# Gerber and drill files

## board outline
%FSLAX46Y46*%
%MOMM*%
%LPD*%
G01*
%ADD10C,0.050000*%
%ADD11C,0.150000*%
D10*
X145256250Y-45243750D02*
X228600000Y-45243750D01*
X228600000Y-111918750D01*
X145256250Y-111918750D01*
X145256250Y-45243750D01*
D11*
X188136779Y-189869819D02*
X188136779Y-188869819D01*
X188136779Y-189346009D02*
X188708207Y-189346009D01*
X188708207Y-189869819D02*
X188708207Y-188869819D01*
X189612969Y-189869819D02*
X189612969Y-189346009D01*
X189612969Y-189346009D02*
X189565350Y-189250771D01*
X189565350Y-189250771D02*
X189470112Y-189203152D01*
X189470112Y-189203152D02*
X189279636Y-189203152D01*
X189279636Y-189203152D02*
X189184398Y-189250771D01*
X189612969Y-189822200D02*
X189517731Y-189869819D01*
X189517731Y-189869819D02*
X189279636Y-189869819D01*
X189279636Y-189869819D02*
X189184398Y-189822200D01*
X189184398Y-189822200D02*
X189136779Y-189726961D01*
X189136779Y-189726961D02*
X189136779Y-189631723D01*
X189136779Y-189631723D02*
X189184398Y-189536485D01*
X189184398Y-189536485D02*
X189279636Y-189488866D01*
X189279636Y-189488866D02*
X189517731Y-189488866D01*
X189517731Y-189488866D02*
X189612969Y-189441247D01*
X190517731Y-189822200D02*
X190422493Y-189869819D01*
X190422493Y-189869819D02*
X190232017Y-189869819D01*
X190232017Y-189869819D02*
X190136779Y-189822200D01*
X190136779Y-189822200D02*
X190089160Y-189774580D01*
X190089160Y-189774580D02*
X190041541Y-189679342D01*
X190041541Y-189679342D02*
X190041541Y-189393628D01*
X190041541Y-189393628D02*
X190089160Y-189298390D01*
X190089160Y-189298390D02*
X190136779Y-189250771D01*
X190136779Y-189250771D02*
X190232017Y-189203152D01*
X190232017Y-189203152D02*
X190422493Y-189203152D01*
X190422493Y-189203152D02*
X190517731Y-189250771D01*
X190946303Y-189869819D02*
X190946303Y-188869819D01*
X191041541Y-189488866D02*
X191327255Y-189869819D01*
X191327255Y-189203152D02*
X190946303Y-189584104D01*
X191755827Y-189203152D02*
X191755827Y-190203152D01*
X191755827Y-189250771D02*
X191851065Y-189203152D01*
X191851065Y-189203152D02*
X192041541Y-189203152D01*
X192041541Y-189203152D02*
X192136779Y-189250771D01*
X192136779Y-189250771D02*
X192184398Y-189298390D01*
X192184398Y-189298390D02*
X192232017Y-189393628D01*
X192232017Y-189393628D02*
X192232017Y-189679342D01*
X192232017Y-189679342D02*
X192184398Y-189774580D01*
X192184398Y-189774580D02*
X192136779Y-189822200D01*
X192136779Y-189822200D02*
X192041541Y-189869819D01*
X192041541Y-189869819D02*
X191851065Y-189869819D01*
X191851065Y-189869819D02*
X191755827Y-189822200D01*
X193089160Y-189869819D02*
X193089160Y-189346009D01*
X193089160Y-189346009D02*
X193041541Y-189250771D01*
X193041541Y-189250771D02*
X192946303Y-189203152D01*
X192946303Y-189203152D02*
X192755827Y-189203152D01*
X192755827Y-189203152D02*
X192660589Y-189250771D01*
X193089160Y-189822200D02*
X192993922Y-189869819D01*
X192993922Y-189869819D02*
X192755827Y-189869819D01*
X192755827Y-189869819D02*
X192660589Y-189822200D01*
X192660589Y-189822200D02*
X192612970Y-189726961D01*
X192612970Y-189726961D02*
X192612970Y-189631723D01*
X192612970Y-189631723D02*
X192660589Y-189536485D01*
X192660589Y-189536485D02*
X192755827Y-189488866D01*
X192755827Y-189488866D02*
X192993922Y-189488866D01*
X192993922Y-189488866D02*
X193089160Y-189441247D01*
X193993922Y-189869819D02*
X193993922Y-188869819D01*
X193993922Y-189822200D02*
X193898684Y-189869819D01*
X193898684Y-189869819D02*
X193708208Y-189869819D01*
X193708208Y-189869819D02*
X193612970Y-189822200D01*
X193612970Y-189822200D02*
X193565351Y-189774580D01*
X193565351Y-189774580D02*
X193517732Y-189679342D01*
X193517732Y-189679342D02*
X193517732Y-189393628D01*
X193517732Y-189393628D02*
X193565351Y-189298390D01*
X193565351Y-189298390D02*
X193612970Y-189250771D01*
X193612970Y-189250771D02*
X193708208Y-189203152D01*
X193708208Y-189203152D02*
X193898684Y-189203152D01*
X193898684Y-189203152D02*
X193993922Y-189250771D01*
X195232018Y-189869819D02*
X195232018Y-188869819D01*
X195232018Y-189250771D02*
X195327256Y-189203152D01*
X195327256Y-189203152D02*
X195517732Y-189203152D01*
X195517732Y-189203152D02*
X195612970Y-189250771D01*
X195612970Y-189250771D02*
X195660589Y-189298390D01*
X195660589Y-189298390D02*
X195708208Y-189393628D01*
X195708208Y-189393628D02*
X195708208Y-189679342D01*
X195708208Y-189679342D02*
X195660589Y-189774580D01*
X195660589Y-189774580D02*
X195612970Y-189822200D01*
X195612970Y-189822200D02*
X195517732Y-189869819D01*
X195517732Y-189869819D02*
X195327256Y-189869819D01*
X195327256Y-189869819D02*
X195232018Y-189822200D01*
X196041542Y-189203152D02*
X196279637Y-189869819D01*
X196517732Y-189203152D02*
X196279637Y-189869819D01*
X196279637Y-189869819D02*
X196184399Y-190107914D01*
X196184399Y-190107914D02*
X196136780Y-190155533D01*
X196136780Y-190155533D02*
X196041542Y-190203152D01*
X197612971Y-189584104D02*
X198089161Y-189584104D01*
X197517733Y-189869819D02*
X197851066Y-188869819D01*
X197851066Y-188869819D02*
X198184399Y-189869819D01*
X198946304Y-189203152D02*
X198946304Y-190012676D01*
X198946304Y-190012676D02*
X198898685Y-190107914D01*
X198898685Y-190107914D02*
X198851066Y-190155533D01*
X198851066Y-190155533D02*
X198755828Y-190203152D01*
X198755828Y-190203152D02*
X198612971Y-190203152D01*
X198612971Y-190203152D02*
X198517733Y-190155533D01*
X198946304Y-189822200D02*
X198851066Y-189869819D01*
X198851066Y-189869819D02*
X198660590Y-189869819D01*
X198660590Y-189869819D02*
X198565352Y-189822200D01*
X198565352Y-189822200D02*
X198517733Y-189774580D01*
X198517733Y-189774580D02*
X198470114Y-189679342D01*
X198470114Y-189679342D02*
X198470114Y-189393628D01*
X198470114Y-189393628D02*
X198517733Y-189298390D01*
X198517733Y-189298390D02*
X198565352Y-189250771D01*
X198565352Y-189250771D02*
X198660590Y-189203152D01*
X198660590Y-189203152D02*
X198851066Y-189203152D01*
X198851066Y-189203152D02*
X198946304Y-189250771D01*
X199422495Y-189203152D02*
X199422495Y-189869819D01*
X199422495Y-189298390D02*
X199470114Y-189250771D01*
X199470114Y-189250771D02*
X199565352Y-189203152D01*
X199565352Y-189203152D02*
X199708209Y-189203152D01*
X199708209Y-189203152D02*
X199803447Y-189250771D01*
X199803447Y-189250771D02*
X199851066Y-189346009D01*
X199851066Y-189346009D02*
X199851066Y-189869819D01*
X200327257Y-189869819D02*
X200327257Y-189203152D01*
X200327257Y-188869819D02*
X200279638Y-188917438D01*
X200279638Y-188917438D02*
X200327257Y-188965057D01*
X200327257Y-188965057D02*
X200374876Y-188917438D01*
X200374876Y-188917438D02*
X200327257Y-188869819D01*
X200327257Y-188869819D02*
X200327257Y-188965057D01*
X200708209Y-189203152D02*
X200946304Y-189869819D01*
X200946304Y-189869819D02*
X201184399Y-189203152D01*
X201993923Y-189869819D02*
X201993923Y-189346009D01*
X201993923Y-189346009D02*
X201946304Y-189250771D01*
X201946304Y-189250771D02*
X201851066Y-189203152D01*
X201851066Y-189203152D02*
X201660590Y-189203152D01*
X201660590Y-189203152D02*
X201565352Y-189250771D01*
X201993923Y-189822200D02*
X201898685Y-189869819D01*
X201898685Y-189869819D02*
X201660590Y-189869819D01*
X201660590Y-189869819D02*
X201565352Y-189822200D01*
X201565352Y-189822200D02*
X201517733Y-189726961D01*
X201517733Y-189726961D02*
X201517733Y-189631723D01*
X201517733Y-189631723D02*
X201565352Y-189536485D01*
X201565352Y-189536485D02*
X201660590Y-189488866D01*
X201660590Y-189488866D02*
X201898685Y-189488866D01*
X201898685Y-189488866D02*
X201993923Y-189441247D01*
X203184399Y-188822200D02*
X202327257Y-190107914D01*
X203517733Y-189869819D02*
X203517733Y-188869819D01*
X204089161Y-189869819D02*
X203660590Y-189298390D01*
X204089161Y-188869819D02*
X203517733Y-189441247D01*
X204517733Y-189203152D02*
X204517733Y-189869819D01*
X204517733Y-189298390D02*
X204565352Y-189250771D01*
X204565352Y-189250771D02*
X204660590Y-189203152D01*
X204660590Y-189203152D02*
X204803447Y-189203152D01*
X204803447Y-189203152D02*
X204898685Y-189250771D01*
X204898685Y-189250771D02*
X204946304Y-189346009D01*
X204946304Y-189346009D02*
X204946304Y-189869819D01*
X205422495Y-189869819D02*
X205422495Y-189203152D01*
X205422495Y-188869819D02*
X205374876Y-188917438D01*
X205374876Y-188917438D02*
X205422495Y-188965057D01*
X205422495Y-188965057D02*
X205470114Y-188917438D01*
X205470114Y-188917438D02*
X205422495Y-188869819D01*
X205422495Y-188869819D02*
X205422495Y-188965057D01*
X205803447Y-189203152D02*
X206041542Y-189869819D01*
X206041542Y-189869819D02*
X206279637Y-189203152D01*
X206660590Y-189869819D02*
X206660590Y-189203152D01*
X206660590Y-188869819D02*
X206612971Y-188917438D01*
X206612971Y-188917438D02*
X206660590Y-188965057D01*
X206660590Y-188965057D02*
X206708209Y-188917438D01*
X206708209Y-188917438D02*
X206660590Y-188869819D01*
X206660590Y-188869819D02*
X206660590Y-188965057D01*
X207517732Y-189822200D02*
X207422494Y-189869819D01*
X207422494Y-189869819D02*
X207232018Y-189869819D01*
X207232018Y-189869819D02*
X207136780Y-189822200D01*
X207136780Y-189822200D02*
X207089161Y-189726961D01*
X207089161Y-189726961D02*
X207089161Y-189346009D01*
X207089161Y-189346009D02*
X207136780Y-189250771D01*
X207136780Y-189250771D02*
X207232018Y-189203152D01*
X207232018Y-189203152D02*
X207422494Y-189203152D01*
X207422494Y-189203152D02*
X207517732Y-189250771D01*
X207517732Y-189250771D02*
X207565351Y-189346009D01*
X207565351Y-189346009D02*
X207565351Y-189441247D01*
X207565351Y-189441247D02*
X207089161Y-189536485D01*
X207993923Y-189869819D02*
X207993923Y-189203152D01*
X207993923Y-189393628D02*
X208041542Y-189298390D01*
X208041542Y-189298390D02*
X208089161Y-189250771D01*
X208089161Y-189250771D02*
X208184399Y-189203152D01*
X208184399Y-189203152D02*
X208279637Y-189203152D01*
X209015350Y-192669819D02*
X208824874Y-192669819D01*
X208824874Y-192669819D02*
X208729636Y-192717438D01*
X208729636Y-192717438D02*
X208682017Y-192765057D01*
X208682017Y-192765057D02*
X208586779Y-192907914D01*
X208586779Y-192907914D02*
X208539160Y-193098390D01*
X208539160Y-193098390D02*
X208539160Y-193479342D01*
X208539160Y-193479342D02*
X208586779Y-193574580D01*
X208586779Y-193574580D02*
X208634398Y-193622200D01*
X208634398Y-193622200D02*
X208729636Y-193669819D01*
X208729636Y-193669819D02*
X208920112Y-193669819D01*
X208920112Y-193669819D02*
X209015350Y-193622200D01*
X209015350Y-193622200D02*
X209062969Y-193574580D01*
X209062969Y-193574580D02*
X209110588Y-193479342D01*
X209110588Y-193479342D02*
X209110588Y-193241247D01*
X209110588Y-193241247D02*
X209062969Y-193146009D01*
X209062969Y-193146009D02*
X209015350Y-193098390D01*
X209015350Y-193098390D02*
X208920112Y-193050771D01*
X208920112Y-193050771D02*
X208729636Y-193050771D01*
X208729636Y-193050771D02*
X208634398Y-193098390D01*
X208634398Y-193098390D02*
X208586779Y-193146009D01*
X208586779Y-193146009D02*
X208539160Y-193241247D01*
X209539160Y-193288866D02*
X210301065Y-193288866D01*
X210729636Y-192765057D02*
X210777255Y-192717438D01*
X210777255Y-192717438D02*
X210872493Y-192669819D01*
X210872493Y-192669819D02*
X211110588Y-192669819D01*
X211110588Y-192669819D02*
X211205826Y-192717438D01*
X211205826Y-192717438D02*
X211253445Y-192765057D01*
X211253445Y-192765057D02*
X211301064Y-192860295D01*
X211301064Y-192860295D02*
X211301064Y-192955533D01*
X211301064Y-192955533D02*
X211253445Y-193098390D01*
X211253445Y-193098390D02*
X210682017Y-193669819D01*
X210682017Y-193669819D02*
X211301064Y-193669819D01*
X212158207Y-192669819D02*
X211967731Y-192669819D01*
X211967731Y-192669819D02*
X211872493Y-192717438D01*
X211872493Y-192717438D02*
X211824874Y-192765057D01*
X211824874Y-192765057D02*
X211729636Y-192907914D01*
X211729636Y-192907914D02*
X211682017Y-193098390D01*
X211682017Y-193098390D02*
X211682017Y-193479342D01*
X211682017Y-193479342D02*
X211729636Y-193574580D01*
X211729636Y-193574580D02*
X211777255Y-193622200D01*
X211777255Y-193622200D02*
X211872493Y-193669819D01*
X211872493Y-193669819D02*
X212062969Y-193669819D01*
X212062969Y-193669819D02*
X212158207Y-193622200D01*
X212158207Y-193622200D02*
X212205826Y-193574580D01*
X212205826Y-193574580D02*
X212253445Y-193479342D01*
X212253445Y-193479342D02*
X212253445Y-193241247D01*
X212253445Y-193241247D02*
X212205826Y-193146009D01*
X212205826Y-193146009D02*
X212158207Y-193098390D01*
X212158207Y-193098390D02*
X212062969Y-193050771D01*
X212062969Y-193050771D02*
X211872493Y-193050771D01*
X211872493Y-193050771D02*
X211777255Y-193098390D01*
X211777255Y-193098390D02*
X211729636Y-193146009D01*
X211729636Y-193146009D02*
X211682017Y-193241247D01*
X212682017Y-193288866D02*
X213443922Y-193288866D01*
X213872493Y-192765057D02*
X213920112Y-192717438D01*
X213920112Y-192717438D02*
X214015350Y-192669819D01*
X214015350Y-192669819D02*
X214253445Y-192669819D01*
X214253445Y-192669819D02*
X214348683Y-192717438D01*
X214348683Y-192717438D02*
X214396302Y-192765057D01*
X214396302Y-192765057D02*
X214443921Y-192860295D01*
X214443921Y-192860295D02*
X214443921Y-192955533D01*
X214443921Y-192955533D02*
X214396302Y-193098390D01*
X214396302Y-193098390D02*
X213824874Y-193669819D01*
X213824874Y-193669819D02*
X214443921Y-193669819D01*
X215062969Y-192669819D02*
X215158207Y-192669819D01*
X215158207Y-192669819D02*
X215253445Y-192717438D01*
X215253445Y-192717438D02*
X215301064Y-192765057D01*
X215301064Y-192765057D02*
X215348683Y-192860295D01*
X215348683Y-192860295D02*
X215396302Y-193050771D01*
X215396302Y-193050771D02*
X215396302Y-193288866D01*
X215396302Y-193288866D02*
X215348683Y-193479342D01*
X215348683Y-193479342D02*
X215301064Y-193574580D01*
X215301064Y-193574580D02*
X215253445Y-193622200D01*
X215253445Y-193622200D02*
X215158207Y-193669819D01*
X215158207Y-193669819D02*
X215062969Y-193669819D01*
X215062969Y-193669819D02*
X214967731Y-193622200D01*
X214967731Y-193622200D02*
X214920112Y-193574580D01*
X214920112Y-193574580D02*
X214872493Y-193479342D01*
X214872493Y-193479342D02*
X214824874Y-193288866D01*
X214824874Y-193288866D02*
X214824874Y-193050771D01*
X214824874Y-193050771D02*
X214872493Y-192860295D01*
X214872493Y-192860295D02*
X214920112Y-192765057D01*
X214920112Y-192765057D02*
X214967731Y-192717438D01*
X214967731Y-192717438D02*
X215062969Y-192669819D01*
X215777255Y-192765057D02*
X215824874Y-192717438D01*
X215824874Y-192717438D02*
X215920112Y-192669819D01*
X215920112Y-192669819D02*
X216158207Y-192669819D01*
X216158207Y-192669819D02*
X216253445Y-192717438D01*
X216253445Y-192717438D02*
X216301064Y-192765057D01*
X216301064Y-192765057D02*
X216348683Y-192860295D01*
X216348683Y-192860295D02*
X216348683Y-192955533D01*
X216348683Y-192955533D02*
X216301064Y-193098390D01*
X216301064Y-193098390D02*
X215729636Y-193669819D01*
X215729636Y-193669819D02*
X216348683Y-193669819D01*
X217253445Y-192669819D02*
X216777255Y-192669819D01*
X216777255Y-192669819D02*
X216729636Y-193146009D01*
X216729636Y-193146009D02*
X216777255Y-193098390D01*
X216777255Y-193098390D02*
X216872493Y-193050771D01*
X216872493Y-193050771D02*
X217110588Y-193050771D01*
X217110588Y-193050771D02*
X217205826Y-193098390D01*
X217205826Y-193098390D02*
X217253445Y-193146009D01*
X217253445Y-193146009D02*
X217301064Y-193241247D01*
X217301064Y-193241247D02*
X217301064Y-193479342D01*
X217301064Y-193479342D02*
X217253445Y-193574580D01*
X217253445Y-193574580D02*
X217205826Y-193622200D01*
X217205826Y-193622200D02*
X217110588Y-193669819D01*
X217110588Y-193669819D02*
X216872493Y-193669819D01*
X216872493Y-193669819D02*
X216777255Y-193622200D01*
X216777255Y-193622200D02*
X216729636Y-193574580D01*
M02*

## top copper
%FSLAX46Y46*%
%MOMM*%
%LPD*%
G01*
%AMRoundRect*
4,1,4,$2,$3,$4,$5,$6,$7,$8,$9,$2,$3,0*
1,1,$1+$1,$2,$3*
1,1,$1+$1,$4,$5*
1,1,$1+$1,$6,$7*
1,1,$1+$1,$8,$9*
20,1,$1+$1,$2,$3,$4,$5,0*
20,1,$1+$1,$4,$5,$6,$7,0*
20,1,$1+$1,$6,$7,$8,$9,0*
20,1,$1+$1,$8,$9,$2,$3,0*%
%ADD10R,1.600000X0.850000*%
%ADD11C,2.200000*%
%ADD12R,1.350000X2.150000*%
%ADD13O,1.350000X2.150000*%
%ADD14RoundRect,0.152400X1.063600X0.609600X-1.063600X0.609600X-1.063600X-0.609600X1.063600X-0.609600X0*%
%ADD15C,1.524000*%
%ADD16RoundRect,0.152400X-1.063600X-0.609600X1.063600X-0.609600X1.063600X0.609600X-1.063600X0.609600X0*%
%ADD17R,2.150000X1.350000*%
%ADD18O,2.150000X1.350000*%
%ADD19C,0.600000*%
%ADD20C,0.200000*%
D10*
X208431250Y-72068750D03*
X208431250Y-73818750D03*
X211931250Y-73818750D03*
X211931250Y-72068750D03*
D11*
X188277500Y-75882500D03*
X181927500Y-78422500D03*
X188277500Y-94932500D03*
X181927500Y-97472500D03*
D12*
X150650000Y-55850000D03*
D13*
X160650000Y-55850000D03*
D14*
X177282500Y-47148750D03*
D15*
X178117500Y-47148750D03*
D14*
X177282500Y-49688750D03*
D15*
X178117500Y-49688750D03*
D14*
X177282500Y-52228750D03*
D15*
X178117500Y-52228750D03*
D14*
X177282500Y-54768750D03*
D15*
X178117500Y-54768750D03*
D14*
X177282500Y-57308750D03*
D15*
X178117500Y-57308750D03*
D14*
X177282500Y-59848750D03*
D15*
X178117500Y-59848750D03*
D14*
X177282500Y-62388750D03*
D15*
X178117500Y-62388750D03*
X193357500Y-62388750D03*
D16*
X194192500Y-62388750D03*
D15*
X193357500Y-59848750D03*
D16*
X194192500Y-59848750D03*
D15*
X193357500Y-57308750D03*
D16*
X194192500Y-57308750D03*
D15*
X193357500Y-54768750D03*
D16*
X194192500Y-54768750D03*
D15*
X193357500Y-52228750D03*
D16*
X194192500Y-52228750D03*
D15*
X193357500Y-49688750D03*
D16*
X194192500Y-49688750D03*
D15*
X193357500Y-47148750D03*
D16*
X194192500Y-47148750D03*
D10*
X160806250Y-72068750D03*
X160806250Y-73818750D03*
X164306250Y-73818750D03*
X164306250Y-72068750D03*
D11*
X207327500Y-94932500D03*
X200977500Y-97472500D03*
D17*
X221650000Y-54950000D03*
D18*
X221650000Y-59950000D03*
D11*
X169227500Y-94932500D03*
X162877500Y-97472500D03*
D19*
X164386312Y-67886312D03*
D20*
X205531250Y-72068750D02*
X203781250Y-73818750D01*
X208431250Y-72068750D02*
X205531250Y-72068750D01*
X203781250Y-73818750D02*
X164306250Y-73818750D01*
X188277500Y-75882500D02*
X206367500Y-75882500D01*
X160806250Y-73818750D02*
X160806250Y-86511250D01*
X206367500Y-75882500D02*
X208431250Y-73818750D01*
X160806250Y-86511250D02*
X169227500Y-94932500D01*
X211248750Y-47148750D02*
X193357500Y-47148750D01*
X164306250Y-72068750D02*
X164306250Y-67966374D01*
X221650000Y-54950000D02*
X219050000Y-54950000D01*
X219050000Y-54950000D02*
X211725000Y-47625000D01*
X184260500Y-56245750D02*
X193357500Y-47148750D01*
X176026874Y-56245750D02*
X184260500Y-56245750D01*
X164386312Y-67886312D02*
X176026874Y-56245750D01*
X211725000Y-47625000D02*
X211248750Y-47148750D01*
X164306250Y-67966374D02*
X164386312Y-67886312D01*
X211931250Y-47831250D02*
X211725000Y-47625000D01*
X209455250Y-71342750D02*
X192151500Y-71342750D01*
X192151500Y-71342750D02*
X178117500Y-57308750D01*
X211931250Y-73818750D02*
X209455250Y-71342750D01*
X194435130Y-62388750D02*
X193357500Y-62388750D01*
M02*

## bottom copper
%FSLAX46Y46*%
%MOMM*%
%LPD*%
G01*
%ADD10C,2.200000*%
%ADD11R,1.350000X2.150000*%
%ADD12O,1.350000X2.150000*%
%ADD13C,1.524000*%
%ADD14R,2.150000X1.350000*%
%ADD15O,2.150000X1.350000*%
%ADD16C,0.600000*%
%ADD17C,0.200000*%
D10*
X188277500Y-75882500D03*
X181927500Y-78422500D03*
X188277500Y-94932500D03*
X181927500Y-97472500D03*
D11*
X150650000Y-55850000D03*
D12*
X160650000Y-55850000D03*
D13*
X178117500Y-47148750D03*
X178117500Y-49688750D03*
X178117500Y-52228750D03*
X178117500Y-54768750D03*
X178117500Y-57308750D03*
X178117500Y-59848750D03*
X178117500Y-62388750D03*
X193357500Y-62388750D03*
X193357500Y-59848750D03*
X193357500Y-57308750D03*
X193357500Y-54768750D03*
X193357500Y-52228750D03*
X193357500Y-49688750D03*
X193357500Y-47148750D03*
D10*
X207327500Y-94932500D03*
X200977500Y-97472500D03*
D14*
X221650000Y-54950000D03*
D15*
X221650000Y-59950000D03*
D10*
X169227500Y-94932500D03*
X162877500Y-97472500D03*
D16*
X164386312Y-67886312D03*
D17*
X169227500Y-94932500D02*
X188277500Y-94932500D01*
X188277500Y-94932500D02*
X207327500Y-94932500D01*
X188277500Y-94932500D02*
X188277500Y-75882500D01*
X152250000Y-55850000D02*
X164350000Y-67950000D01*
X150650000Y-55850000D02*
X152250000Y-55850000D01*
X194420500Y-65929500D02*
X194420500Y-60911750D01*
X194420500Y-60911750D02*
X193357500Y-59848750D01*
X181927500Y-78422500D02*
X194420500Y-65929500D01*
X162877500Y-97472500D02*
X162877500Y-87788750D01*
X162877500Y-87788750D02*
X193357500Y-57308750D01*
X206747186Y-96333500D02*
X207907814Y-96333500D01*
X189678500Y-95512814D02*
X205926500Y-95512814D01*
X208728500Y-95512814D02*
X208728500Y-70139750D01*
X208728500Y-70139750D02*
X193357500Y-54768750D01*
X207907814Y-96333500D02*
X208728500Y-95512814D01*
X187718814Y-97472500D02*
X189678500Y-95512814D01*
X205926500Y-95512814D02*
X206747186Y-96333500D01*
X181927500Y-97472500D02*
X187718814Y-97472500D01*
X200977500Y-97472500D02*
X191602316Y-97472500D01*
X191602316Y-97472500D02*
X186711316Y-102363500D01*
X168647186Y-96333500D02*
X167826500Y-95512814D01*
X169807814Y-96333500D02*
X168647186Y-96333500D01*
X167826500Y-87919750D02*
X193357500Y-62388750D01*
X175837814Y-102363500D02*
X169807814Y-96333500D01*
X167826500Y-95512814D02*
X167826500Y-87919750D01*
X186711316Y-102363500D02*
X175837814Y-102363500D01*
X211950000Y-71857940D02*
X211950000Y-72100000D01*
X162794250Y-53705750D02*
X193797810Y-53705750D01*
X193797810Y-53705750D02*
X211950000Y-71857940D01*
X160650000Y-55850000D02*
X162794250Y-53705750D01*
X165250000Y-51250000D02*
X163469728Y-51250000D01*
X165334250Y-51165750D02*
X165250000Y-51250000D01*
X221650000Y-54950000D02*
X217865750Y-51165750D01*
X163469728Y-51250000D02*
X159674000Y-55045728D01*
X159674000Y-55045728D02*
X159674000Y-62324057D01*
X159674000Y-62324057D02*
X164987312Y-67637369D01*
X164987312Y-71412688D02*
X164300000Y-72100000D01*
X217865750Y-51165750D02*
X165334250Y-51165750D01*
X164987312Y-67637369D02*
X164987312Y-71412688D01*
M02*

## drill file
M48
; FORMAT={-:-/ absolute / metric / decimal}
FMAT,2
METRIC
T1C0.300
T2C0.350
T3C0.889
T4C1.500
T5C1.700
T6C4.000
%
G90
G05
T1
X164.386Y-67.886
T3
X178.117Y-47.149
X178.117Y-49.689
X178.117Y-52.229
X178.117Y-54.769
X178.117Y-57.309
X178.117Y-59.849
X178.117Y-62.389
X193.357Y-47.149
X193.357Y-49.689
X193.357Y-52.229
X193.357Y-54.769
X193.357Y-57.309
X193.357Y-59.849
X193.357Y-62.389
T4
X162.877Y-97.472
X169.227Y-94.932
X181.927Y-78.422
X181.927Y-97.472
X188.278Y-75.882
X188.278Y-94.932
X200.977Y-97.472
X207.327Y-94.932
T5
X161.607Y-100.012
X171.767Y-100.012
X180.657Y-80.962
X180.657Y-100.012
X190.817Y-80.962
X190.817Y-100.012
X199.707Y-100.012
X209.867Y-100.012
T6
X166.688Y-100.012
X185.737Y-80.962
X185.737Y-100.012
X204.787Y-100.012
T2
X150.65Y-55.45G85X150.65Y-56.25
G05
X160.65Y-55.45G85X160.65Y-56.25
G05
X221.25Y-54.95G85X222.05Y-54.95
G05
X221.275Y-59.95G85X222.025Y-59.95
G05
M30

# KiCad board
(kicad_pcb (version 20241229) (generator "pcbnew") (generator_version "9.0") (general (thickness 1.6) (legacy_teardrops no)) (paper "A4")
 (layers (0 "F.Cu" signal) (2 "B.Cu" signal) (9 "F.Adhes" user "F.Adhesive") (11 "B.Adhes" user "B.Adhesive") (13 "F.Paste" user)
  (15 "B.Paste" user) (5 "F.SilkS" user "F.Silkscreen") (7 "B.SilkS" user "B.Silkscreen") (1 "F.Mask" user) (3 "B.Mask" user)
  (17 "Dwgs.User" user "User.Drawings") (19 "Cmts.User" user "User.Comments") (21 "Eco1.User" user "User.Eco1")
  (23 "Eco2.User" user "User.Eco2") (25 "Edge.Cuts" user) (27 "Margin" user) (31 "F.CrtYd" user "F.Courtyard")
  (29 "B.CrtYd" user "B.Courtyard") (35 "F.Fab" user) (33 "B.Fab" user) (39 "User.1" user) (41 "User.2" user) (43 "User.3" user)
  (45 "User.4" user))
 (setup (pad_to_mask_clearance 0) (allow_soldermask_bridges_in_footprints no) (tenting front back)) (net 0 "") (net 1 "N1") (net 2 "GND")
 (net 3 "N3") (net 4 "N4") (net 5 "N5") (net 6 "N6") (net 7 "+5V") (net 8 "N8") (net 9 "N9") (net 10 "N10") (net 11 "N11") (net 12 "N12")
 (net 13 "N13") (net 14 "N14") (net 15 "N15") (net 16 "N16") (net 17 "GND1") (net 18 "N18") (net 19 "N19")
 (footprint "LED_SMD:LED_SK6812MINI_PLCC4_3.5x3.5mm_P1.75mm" (layer "F.Cu") (at 210.18125 72.94375)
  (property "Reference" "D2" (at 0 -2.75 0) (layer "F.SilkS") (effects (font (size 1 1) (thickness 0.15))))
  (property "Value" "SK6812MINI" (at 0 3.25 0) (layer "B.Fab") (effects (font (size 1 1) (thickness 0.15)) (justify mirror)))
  (pad "1" smd rect (at -1.75 -0.875) (size 1.6 0.85) (layers "F.Cu" "F.Mask" "F.Paste") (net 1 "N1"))
  (pad "2" smd rect (at -1.75 0.875) (size 1.6 0.85) (layers "F.Cu" "F.Mask" "F.Paste") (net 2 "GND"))
  (pad "3" smd rect (at 1.75 0.875) (size 1.6 0.85) (layers "F.Cu" "F.Mask" "F.Paste") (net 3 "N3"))
  (pad "4" smd rect (at 1.75 -0.875) (size 1.6 0.85) (layers "F.Cu" "F.Mask" "F.Paste") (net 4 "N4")))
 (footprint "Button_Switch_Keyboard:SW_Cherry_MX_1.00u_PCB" (layer "F.Cu") (at 188.2775 75.8825)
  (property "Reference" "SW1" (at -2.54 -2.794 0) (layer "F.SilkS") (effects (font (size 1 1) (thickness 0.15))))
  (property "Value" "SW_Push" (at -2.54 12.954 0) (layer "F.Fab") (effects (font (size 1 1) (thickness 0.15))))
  (pad "" np_thru_hole circle (at -7.62 5.08) (size 1.7 1.7) (drill 1.7) (layers "*.Cu" "*.Mask"))
  (pad "" np_thru_hole circle (at -2.54 5.08) (size 4 4) (drill 4) (layers "*.Cu" "*.Mask"))
  (pad "" np_thru_hole circle (at 2.54 5.08) (size 1.7 1.7) (drill 1.7) (layers "*.Cu" "*.Mask"))
  (pad "1" thru_hole circle (at 0 0) (size 2.2 2.2) (drill 1.5) (layers "*.Cu" "*.Mask") (remove_unused_layers no) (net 2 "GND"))
  (pad "2" thru_hole circle (at -6.35 2.54) (size 2.2 2.2) (drill 1.5) (layers "*.Cu" "*.Mask") (remove_unused_layers no) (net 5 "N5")))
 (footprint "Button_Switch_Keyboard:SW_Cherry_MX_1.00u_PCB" (layer "F.Cu") (at 188.2775 94.9325)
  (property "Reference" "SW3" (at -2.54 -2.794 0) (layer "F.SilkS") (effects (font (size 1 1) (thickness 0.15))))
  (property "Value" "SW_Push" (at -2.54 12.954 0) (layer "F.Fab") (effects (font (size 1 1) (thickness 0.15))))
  (pad "" np_thru_hole circle (at -7.62 5.08) (size 1.7 1.7) (drill 1.7) (layers "*.Cu" "*.Mask"))
  (pad "" np_thru_hole circle (at -2.54 5.08) (size 4 4) (drill 4) (layers "*.Cu" "*.Mask"))
  (pad "" np_thru_hole circle (at 2.54 5.08) (size 1.7 1.7) (drill 1.7) (layers "*.Cu" "*.Mask"))
  (pad "1" thru_hole circle (at 0 0) (size 2.2 2.2) (drill 1.5) (layers "*.Cu" "*.Mask") (remove_unused_layers no) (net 2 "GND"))
  (pad "2" thru_hole circle (at -6.35 2.54) (size 2.2 2.2) (drill 1.5) (layers "*.Cu" "*.Mask") (remove_unused_layers no) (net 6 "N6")))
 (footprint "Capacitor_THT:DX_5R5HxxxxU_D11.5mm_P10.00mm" (layer "F.Cu") (at 150.65 55.85)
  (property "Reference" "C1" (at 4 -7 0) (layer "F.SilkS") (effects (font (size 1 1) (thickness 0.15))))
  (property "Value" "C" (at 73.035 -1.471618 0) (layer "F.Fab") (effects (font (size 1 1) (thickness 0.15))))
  (pad "1" thru_hole rect (at 0 0) (size 1.35 2.15) (drill oval 0.35 1.15) (layers "*.Cu" "*.Mask") (remove_unused_layers no) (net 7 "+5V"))
  (pad "2" thru_hole oval (at 10 0) (size 1.35 2.15) (drill oval 0.35 1.15) (layers "*.Cu" "*.Mask") (remove_unused_layers no) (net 4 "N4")))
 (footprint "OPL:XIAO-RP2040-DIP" (layer "F.Cu") (at 185.7375 54.76875)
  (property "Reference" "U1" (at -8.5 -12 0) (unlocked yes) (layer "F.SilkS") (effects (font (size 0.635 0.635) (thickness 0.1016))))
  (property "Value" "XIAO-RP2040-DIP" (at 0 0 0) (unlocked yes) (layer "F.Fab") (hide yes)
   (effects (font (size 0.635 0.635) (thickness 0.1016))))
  (pad "1" smd roundrect (at -8.455 -7.62 180) (size 2.432 1.524) (layers "F.Cu" "F.Mask") (roundrect_rratio 0.1) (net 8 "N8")
   (thermal_bridge_angle 45))
  (pad "1" thru_hole circle (at -7.62 -7.62 180) (size 1.524 1.524) (drill 0.889) (layers "*.Cu" "*.Mask") (remove_unused_layers no)
   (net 8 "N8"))
  (pad "2" smd roundrect (at -8.455 -5.08 180) (size 2.432 1.524) (layers "F.Cu" "F.Mask") (roundrect_rratio 0.1) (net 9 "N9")
   (thermal_bridge_angle 45))
  (pad "2" thru_hole circle (at -7.62 -5.08 180) (size 1.524 1.524) (drill 0.889) (layers "*.Cu" "*.Mask") (remove_unused_layers no)
   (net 9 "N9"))
  (pad "3" smd roundrect (at -8.455 -2.54 180) (size 2.432 1.524) (layers "F.Cu" "F.Mask") (roundrect_rratio 0.1) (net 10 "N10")
   (thermal_bridge_angle 45))
  (pad "3" thru_hole circle (at -7.62 -2.54 180) (size 1.524 1.524) (drill 0.889) (layers "*.Cu" "*.Mask") (remove_unused_layers no)
   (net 10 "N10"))
  (pad "4" smd roundrect (at -8.455 0 180) (size 2.432 1.524) (layers "F.Cu" "F.Mask") (roundrect_rratio 0.1) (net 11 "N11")
   (thermal_bridge_angle 45))
  (pad "4" thru_hole circle (at -7.62 0 180) (size 1.524 1.524) (drill 0.889) (layers "*.Cu" "*.Mask") (remove_unused_layers no)
   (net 11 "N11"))
  (pad "5" smd roundrect (at -8.455 2.54 180) (size 2.432 1.524) (layers "F.Cu" "F.Mask") (roundrect_rratio 0.1) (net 3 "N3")
   (thermal_bridge_angle 45))
  (pad "5" thru_hole circle (at -7.62 2.54 180) (size 1.524 1.524) (drill 0.889) (layers "*.Cu" "*.Mask") (remove_unused_layers no)
   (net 3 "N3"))
  (pad "6" smd roundrect (at -8.455 5.08 180) (size 2.432 1.524) (layers "F.Cu" "F.Mask") (roundrect_rratio 0.1) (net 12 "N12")
   (thermal_bridge_angle 45))
  (pad "6" thru_hole circle (at -7.62 5.08 180) (size 1.524 1.524) (drill 0.889) (layers "*.Cu" "*.Mask") (remove_unused_layers no)
   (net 12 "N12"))
  (pad "7" smd roundrect (at -8.455 7.62 180) (size 2.432 1.524) (layers "F.Cu" "F.Mask") (roundrect_rratio 0.1) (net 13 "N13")
   (thermal_bridge_angle 45))
  (pad "7" thru_hole circle (at -7.62 7.62 180) (size 1.524 1.524) (drill 0.889) (layers "*.Cu" "*.Mask") (remove_unused_layers no)
   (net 13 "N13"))
  (pad "8" thru_hole circle (at 7.62 7.62) (size 1.524 1.524) (drill 0.889) (layers "*.Cu" "*.Mask") (remove_unused_layers no)
   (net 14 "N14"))
  (pad "8" smd roundrect (at 8.455 7.62) (size 2.432 1.524) (layers "F.Cu" "F.Mask") (roundrect_rratio 0.1) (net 14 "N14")
   (thermal_bridge_angle 45))
  (pad "9" thru_hole circle (at 7.62 5.08) (size 1.524 1.524) (drill 0.889) (layers "*.Cu" "*.Mask") (remove_unused_layers no) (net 5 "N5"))
  (pad "9" smd roundrect (at 8.455 5.08) (size 2.432 1.524) (layers "F.Cu" "F.Mask") (roundrect_rratio 0.1) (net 5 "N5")
   (thermal_bridge_angle 45))
  (pad "10" thru_hole circle (at 7.62 2.54) (size 1.524 1.524) (drill 0.889) (layers "*.Cu" "*.Mask") (remove_unused_layers no)
   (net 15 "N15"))
  (pad "10" smd roundrect (at 8.455 2.54) (size 2.432 1.524) (layers "F.Cu" "F.Mask") (roundrect_rratio 0.1) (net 15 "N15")
   (thermal_bridge_angle 45))
  (pad "11" thru_hole circle (at 7.62 0) (size 1.524 1.524) (drill 0.889) (layers "*.Cu" "*.Mask") (remove_unused_layers no) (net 6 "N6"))
  (pad "11" smd roundrect (at 8.455 0) (size 2.432 1.524) (layers "F.Cu" "F.Mask") (roundrect_rratio 0.1) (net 6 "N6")
   (thermal_bridge_angle 45))
  (pad "12" thru_hole circle (at 7.62 -2.54) (size 1.524 1.524) (drill 0.889) (layers "*.Cu" "*.Mask") (remove_unused_layers no)
   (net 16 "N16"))
  (pad "12" smd roundrect (at 8.455 -2.54) (size 2.432 1.524) (layers "F.Cu" "F.Mask") (roundrect_rratio 0.1) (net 16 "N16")
   (thermal_bridge_angle 45))
  (pad "13" thru_hole circle (at 7.62 -5.08) (size 1.524 1.524) (drill 0.889) (layers "*.Cu" "*.Mask") (remove_unused_layers no)
   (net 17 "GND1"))
  (pad "13" smd roundrect (at 8.455 -5.08) (size 2.432 1.524) (layers "F.Cu" "F.Mask") (roundrect_rratio 0.1) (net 17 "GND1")
   (thermal_bridge_angle 45))
  (pad "14" thru_hole circle (at 7.62 -7.62) (size 1.524 1.524) (drill 0.889) (layers "*.Cu" "*.Mask") (remove_unused_layers no)
   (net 7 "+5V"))
  (pad "14" smd roundrect (at 8.455 -7.62) (size 2.432 1.524) (layers "F.Cu" "F.Mask") (roundrect_rratio 0.1) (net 7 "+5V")
   (thermal_bridge_angle 45)))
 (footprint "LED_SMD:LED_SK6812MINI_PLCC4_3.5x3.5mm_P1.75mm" (layer "F.Cu") (at 162.55625 72.94375)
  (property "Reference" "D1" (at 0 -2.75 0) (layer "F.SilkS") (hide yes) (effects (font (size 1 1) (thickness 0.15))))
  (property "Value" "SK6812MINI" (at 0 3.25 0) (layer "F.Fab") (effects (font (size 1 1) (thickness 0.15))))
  (pad "1" smd rect (at -1.75 -0.875) (size 1.6 0.85) (layers "F.Cu" "F.Mask" "F.Paste") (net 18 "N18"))
  (pad "2" smd rect (at -1.75 0.875) (size 1.6 0.85) (layers "F.Cu" "F.Mask" "F.Paste") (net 2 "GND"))
  (pad "3" smd rect (at 1.75 0.875) (size 1.6 0.85) (layers "F.Cu" "F.Mask" "F.Paste") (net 1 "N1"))
  (pad "4" smd rect (at 1.75 -0.875) (size 1.6 0.85) (layers "F.Cu" "F.Mask" "F.Paste") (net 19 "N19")))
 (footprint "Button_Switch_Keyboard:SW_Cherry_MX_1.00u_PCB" (layer "F.Cu") (at 207.3275 94.9325)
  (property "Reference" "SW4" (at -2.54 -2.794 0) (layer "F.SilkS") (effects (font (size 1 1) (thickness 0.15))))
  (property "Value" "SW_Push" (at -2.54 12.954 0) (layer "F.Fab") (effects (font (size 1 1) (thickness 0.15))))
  (pad "" np_thru_hole circle (at -7.62 5.08) (size 1.7 1.7) (drill 1.7) (layers "*.Cu" "*.Mask"))
  (pad "" np_thru_hole circle (at -2.54 5.08) (size 4 4) (drill 4) (layers "*.Cu" "*.Mask"))
  (pad "" np_thru_hole circle (at 2.54 5.08) (size 1.7 1.7) (drill 1.7) (layers "*.Cu" "*.Mask"))
  (pad "1" thru_hole circle (at 0 0) (size 2.2 2.2) (drill 1.5) (layers "*.Cu" "*.Mask") (remove_unused_layers no) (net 2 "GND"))
  (pad "2" thru_hole circle (at -6.35 2.54) (size 2.2 2.2) (drill 1.5) (layers "*.Cu" "*.Mask") (remove_unused_layers no) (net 14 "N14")))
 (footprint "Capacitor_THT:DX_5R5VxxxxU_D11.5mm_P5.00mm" (layer "F.Cu") (at 221.65 54.95)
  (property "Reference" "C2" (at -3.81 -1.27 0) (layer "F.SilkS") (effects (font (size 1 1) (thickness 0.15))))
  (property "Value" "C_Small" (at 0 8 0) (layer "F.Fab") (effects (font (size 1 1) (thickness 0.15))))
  (pad "1" thru_hole rect (at 0 0) (size 2.15 1.35) (drill oval 1.15 0.35) (layers "*.Cu" "*.Mask") (remove_unused_layers no) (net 19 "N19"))
  (pad "2" thru_hole oval (at 0 5) (size 2.15 1.35) (drill oval 1.1 0.35) (layers "*.Cu" "*.Mask") (remove_unused_layers no) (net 7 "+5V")))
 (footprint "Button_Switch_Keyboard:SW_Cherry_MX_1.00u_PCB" (layer "F.Cu") (at 169.2275 94.9325)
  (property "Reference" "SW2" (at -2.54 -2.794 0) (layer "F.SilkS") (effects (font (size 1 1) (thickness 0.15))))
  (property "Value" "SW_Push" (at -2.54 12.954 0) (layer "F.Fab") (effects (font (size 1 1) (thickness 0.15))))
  (pad "" np_thru_hole circle (at -7.62 5.08) (size 1.7 1.7) (drill 1.7) (layers "*.Cu" "*.Mask"))
  (pad "" np_thru_hole circle (at -2.54 5.08) (size 4 4) (drill 4) (layers "*.Cu" "*.Mask"))
  (pad "" np_thru_hole circle (at 2.54 5.08) (size 1.7 1.7) (drill 1.7) (layers "*.Cu" "*.Mask"))
  (pad "1" thru_hole circle (at 0 0) (size 2.2 2.2) (drill 1.5) (layers "*.Cu" "*.Mask") (remove_unused_layers no) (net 2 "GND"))
  (pad "2" thru_hole circle (at -6.35 2.54) (size 2.2 2.2) (drill 1.5) (layers "*.Cu" "*.Mask") (remove_unused_layers no) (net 15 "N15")))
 (gr_rect (start 145.25625 45.24375) (end 228.6 111.91875) (stroke (width 0.05) (type default)) (fill no) (layer "Edge.Cuts"))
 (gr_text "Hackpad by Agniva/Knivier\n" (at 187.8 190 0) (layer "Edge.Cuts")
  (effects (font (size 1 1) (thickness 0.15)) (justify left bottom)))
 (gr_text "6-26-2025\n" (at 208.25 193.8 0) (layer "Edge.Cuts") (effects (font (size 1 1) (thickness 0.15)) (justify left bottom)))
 (segment (start 205.53125 72.06875) (end 203.78125 73.81875) (width 0.2) (layer "F.Cu") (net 1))
 (segment (start 208.43125 72.06875) (end 205.53125 72.06875) (width 0.2) (layer "F.Cu") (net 1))
 (segment (start 203.78125 73.81875) (end 164.30625 73.81875) (width 0.2) (layer "F.Cu") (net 1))
 (segment (start 188.2775 75.8825) (end 206.3675 75.8825) (width 0.2) (layer "F.Cu") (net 2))
 (segment (start 160.80625 73.81875) (end 160.80625 86.51125) (width 0.2) (layer "F.Cu") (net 2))
 (segment (start 206.3675 75.8825) (end 208.43125 73.81875) (width 0.2) (layer "F.Cu") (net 2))
 (segment (start 160.80625 86.51125) (end 169.2275 94.9325) (width 0.2) (layer "F.Cu") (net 2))
 (segment (start 169.2275 94.9325) (end 188.2775 94.9325) (width 0.2) (layer "B.Cu") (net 2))
 (segment (start 188.2775 94.9325) (end 207.3275 94.9325) (width 0.2) (layer "B.Cu") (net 2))
 (segment (start 188.2775 94.9325) (end 188.2775 75.8825) (width 0.2) (layer "B.Cu") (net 2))
 (segment (start 211.24875 47.14875) (end 193.3575 47.14875) (width 0.2) (layer "F.Cu") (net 7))
 (segment (start 164.30625 72.06875) (end 164.30625 67.966374) (width 0.2) (layer "F.Cu") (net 7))
 (segment (start 221.65 54.95) (end 219.05 54.95) (width 0.2) (layer "F.Cu") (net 7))
 (segment (start 219.05 54.95) (end 211.725 47.625) (width 0.2) (layer "F.Cu") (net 7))
 (segment (start 184.2605 56.24575) (end 193.3575 47.14875) (width 0.2) (layer "F.Cu") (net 7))
 (segment (start 176.026874 56.24575) (end 184.2605 56.24575) (width 0.2) (layer "F.Cu") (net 7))
 (segment (start 164.386312 67.886312) (end 176.026874 56.24575) (width 0.2) (layer "F.Cu") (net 7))
 (segment (start 211.725 47.625) (end 211.24875 47.14875) (width 0.2) (layer "F.Cu") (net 7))
 (segment (start 164.30625 67.966374) (end 164.386312 67.886312) (width 0.2) (layer "F.Cu") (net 7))
 (segment (start 211.93125 47.83125) (end 211.725 47.625) (width 0.2) (layer "F.Cu") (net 7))
 (via (at 164.386312 67.886312) (size 0.6) (drill 0.3) (layers "F.Cu" "B.Cu") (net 7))
 (segment (start 152.25 55.85) (end 164.35 67.95) (width 0.2) (layer "B.Cu") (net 7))
 (segment (start 150.65 55.85) (end 152.25 55.85) (width 0.2) (layer "B.Cu") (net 7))
 (segment (start 209.45525 71.34275) (end 192.1515 71.34275) (width 0.2) (layer "F.Cu") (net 3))
 (segment (start 192.1515 71.34275) (end 178.1175 57.30875) (width 0.2) (layer "F.Cu") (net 3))
 (segment (start 211.93125 73.81875) (end 209.45525 71.34275) (width 0.2) (layer "F.Cu") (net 3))
 (segment (start 194.4205 65.9295) (end 194.4205 60.91175) (width 0.2) (layer "B.Cu") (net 5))
 (segment (start 194.4205 60.91175) (end 193.3575 59.84875) (width 0.2) (layer "B.Cu") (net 5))
 (segment (start 181.9275 78.4225) (end 194.4205 65.9295) (width 0.2) (layer "B.Cu") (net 5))
 (segment (start 162.8775 97.4725) (end 162.8775 87.78875) (width 0.2) (layer "B.Cu") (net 15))
 (segment (start 162.8775 87.78875) (end 193.3575 57.30875) (width 0.2) (layer "B.Cu") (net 15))
 (segment (start 206.747186 96.3335) (end 207.907814 96.3335) (width 0.2) (layer "B.Cu") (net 6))
 (segment (start 189.6785 95.512814) (end 205.9265 95.512814) (width 0.2) (layer "B.Cu") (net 6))
 (segment (start 208.7285 95.512814) (end 208.7285 70.13975) (width 0.2) (layer "B.Cu") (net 6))
 (segment (start 208.7285 70.13975) (end 193.3575 54.76875) (width 0.2) (layer "B.Cu") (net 6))
 (segment (start 207.907814 96.3335) (end 208.7285 95.512814) (width 0.2) (layer "B.Cu") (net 6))
 (segment (start 187.718814 97.4725) (end 189.6785 95.512814) (width 0.2) (layer "B.Cu") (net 6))
 (segment (start 205.9265 95.512814) (end 206.747186 96.3335) (width 0.2) (layer "B.Cu") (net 6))
 (segment (start 181.9275 97.4725) (end 187.718814 97.4725) (width 0.2) (layer "B.Cu") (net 6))
 (segment (start 194.43513 62.38875) (end 193.3575 62.38875) (width 0.2) (layer "F.Cu") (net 14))
 (segment (start 200.9775 97.4725) (end 191.602316 97.4725) (width 0.2) (layer "B.Cu") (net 14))
 (segment (start 191.602316 97.4725) (end 186.711316 102.3635) (width 0.2) (layer "B.Cu") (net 14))
 (segment (start 168.647186 96.3335) (end 167.8265 95.512814) (width 0.2) (layer "B.Cu") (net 14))
 (segment (start 169.807814 96.3335) (end 168.647186 96.3335) (width 0.2) (layer "B.Cu") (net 14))
 (segment (start 167.8265 87.91975) (end 193.3575 62.38875) (width 0.2) (layer "B.Cu") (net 14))
 (segment (start 175.837814 102.3635) (end 169.807814 96.3335) (width 0.2) (layer "B.Cu") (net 14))
 (segment (start 167.8265 95.512814) (end 167.8265 87.91975) (width 0.2) (layer "B.Cu") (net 14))
 (segment (start 186.711316 102.3635) (end 175.837814 102.3635) (width 0.2) (layer "B.Cu") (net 14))
 (segment (start 211.95 71.85794) (end 211.95 72.1) (width 0.2) (layer "B.Cu") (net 4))
 (segment (start 162.79425 53.70575) (end 193.79781 53.70575) (width 0.2) (layer "B.Cu") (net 4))
 (segment (start 193.79781 53.70575) (end 211.95 71.85794) (width 0.2) (layer "B.Cu") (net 4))
 (segment (start 160.65 55.85) (end 162.79425 53.70575) (width 0.2) (layer "B.Cu") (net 4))
 (segment (start 165.25 51.25) (end 163.469728 51.25) (width 0.2) (layer "B.Cu") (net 19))
 (segment (start 165.33425 51.16575) (end 165.25 51.25) (width 0.2) (layer "B.Cu") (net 19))
 (segment (start 221.65 54.95) (end 217.86575 51.16575) (width 0.2) (layer "B.Cu") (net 19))
 (segment (start 163.469728 51.25) (end 159.674 55.045728) (width 0.2) (layer "B.Cu") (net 19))
 (segment (start 159.674 55.045728) (end 159.674 62.324057) (width 0.2) (layer "B.Cu") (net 19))
 (segment (start 159.674 62.324057) (end 164.987312 67.637369) (width 0.2) (layer "B.Cu") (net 19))
 (segment (start 164.987312 71.412688) (end 164.3 72.1) (width 0.2) (layer "B.Cu") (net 19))
 (segment (start 217.86575 51.16575) (end 165.33425 51.16575) (width 0.2) (layer "B.Cu") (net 19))
 (segment (start 164.987312 67.637369) (end 164.987312 71.412688) (width 0.2) (layer "B.Cu") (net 19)))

